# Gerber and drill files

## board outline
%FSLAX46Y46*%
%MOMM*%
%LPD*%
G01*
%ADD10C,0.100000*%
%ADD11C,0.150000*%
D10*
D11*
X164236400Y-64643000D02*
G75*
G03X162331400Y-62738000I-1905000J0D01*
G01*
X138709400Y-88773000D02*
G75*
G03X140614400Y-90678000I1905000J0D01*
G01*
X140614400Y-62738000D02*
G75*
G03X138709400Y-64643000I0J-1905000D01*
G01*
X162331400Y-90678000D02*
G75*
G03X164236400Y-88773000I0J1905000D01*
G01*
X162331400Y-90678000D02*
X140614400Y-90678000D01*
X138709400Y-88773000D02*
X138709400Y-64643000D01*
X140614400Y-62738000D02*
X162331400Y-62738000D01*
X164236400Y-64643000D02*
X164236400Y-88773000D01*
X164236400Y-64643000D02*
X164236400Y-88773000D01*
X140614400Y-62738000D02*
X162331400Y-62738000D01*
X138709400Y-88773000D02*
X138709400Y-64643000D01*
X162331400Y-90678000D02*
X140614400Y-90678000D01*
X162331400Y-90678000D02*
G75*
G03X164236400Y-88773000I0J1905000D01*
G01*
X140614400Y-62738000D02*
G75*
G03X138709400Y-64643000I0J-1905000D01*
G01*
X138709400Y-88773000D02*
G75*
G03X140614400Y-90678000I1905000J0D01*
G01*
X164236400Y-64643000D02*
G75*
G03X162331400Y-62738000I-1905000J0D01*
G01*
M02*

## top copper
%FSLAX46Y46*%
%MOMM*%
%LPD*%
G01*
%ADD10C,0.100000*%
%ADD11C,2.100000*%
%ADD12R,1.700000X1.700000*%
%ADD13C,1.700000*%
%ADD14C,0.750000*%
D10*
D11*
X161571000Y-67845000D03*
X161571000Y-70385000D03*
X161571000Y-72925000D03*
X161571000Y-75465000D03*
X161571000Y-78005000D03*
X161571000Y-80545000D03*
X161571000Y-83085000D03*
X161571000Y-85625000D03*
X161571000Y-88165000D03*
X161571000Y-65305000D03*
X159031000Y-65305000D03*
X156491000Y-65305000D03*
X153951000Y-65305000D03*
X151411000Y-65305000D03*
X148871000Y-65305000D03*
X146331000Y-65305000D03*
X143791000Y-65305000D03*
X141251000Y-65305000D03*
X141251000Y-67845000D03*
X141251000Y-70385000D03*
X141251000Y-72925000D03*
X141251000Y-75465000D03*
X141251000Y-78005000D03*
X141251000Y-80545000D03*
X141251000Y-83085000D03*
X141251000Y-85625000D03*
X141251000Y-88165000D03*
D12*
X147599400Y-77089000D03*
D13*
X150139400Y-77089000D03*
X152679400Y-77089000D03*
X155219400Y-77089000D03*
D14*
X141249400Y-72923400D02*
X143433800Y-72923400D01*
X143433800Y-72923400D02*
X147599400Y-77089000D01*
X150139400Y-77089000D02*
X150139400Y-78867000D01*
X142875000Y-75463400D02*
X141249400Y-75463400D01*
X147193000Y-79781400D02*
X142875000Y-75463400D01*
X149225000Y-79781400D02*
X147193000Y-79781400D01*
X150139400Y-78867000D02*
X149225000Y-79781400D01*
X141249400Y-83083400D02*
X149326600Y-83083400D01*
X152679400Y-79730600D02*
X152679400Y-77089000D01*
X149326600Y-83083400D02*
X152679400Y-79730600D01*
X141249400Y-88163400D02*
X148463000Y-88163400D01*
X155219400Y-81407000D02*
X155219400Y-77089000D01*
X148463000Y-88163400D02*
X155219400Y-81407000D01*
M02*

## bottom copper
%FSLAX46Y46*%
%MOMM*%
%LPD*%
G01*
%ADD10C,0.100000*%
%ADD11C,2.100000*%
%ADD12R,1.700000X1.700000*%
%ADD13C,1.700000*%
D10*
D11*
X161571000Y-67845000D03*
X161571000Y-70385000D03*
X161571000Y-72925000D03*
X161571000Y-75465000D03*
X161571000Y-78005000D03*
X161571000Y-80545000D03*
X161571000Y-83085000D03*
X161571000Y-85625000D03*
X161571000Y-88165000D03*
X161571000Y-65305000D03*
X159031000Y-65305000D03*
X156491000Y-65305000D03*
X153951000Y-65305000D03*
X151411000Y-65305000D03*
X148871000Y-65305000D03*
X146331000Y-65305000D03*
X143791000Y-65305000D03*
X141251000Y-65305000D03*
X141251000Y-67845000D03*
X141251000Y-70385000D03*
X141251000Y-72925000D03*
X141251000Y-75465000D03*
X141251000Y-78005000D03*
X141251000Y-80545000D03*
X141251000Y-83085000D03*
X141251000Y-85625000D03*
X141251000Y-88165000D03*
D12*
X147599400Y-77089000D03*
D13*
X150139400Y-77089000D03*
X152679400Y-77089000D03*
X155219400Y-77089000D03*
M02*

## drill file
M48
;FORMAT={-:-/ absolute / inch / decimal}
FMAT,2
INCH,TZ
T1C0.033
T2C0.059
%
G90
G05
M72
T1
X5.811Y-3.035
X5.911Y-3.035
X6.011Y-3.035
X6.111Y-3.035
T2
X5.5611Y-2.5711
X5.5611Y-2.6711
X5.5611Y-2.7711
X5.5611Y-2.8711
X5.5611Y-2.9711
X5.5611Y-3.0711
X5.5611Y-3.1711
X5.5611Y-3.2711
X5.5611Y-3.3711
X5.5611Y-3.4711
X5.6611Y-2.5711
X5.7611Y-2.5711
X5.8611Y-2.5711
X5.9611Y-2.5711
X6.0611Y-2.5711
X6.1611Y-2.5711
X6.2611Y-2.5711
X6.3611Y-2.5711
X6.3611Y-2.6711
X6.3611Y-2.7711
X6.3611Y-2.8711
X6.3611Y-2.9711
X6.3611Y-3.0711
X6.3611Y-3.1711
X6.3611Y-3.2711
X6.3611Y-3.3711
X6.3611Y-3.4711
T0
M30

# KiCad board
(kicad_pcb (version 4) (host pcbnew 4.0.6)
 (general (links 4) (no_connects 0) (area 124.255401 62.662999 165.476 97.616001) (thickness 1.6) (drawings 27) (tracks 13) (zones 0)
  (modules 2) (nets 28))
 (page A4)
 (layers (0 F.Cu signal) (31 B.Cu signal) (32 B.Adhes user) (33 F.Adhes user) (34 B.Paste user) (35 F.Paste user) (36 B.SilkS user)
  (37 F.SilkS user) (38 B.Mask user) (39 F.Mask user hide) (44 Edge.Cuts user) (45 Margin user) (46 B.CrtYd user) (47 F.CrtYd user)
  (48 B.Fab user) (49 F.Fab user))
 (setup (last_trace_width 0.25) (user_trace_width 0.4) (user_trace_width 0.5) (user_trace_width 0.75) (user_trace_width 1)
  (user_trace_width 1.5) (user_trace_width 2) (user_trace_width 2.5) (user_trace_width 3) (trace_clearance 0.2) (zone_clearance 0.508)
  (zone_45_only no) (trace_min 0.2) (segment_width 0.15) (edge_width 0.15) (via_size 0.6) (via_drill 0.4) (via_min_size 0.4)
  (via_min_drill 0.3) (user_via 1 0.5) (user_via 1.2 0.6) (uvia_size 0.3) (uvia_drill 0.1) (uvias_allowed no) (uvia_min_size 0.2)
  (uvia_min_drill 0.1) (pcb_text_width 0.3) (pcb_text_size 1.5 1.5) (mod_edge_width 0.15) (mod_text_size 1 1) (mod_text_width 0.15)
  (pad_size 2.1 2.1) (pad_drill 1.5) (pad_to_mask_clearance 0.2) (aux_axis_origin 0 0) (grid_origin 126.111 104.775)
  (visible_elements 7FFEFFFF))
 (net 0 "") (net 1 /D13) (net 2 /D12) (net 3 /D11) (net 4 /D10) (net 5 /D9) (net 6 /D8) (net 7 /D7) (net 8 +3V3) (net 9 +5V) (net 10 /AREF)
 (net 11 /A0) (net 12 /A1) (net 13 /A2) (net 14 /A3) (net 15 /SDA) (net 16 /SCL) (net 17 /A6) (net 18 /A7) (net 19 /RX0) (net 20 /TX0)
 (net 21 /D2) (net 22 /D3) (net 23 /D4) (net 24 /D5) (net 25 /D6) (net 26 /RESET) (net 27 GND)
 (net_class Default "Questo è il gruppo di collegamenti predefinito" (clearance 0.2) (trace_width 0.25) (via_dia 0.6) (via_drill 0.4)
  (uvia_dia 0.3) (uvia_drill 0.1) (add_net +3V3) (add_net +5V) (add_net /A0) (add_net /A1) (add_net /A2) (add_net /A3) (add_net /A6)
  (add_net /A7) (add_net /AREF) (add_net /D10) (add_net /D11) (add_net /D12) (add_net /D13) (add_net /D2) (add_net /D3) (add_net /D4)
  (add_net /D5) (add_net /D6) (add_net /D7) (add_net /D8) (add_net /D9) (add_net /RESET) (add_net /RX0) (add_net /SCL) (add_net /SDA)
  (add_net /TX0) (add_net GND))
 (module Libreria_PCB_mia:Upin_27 (layer B.Cu) (at 161.571 88.165 180)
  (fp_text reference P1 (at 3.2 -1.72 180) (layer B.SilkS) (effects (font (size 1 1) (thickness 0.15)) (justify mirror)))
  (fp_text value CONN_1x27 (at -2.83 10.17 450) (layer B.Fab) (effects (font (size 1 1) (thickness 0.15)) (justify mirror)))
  (pad 9 thru_hole circle (at 0 20.32 180) (size 2.1 2.1) (drill 1.5) (layers *.Cu *.Mask) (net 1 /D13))
  (pad 8 thru_hole circle (at 0 17.78 180) (size 2.1 2.1) (drill 1.5) (layers *.Cu *.Mask) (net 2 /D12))
  (pad 7 thru_hole circle (at 0 15.24 180) (size 2.1 2.1) (drill 1.5) (layers *.Cu *.Mask) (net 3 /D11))
  (pad 6 thru_hole circle (at 0 12.7 180) (size 2.1 2.1) (drill 1.5) (layers *.Cu *.Mask) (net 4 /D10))
  (pad 5 thru_hole circle (at 0 10.16 180) (size 2.1 2.1) (drill 1.5) (layers *.Cu *.Mask) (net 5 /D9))
  (pad 4 thru_hole circle (at 0 7.62 180) (size 2.1 2.1) (drill 1.5) (layers *.Cu *.Mask) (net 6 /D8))
  (pad 3 thru_hole circle (at 0 5.08 180) (size 2.1 2.1) (drill 1.5) (layers *.Cu *.Mask) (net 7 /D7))
  (pad 2 thru_hole circle (at 0 2.54 180) (size 2.1 2.1) (drill 1.5) (layers *.Cu *.Mask) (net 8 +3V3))
  (pad 1 thru_hole circle (at 0 0 180) (size 2.1 2.1) (drill 1.5) (layers *.Cu *.Mask) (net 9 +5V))
  (pad 10 thru_hole circle (at 0 22.86 180) (size 2.1 2.1) (drill 1.5) (layers *.Cu *.Mask) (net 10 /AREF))
  (pad 11 thru_hole circle (at 2.54 22.86 180) (size 2.1 2.1) (drill 1.5) (layers *.Cu *.Mask) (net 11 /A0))
  (pad 12 thru_hole circle (at 5.08 22.86 180) (size 2.1 2.1) (drill 1.5) (layers *.Cu *.Mask) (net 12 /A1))
  (pad 13 thru_hole circle (at 7.62 22.86 180) (size 2.1 2.1) (drill 1.5) (layers *.Cu *.Mask) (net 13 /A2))
  (pad 14 thru_hole circle (at 10.16 22.86 180) (size 2.1 2.1) (drill 1.5) (layers *.Cu *.Mask) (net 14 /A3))
  (pad 15 thru_hole circle (at 12.7 22.86 180) (size 2.1 2.1) (drill 1.5) (layers *.Cu *.Mask) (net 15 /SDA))
  (pad 16 thru_hole circle (at 15.24 22.86 180) (size 2.1 2.1) (drill 1.5) (layers *.Cu *.Mask) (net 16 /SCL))
  (pad 17 thru_hole circle (at 17.78 22.86 180) (size 2.1 2.1) (drill 1.5) (layers *.Cu *.Mask) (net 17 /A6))
  (pad 18 thru_hole circle (at 20.32 22.86 180) (size 2.1 2.1) (drill 1.5) (layers *.Cu *.Mask) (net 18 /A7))
  (pad 19 thru_hole circle (at 20.32 20.32 180) (size 2.1 2.1) (drill 1.5) (layers *.Cu *.Mask) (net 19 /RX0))
  (pad 20 thru_hole circle (at 20.32 17.78 180) (size 2.1 2.1) (drill 1.5) (layers *.Cu *.Mask) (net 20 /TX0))
  (pad 21 thru_hole circle (at 20.32 15.24 180) (size 2.1 2.1) (drill 1.5) (layers *.Cu *.Mask) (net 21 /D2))
  (pad 22 thru_hole circle (at 20.32 12.7 180) (size 2.1 2.1) (drill 1.5) (layers *.Cu *.Mask) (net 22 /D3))
  (pad 23 thru_hole circle (at 20.32 10.16 180) (size 2.1 2.1) (drill 1.5) (layers *.Cu *.Mask) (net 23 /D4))
  (pad 24 thru_hole circle (at 20.32 7.62 180) (size 2.1 2.1) (drill 1.5) (layers *.Cu *.Mask) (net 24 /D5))
  (pad 25 thru_hole circle (at 20.32 5.08 180) (size 2.1 2.1) (drill 1.5) (layers *.Cu *.Mask) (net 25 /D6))
  (pad 26 thru_hole circle (at 20.32 2.54 180) (size 2.1 2.1) (drill 1.5) (layers *.Cu *.Mask) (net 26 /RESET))
  (pad 27 thru_hole circle (at 20.32 0 180) (size 2.1 2.1) (drill 1.5) (layers *.Cu *.Mask) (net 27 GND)))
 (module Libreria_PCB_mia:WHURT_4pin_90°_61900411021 (layer F.Cu) (at 147.5994 77.089)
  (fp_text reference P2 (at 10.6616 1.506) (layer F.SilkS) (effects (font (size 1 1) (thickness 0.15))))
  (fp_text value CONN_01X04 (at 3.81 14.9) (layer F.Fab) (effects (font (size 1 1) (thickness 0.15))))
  (pad 1 thru_hole rect (at 0 0) (size 1.7 1.7) (drill 0.85) (layers *.Cu *.Mask) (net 21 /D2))
  (pad 2 thru_hole circle (at 2.54 0) (size 1.7 1.7) (drill 0.85) (layers *.Cu *.Mask) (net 22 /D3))
  (pad 3 thru_hole circle (at 5.08 0) (size 1.7 1.7) (drill 0.85) (layers *.Cu *.Mask) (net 25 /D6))
  (pad 4 thru_hole circle (at 7.62 0) (size 1.7 1.7) (drill 0.85) (layers *.Cu *.Mask) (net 27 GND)))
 (gr_arc (start 162.3314 64.643) (end 162.3314 62.738) (angle 90) (layer Edge.Cuts) (width 0.15))
 (gr_arc (start 140.6144 88.773) (end 140.6144 90.678) (angle 90) (layer Edge.Cuts) (width 0.15))
 (gr_arc (start 140.6144 64.643) (end 138.7094 64.643) (angle 90) (layer Edge.Cuts) (width 0.15))
 (gr_arc (start 162.3314 88.773) (end 164.2364 88.773) (angle 90) (layer Edge.Cuts) (width 0.15))
 (gr_line (start 162.3314 90.678) (end 140.6144 90.678) (angle 90) (layer Edge.Cuts) (width 0.15))
 (gr_line (start 138.7094 88.773) (end 138.7094 64.643) (angle 90) (layer Edge.Cuts) (width 0.15))
 (gr_line (start 140.6144 62.738) (end 162.3314 62.738) (angle 90) (layer Edge.Cuts) (width 0.15))
 (gr_line (start 164.2364 64.643) (end 164.2364 88.773) (angle 90) (layer Edge.Cuts) (width 0.15))
 (gr_line (start 164.2364 64.643) (end 164.2364 88.773) (angle 90) (layer Edge.Cuts) (width 0.15))
 (gr_line (start 140.6144 62.738) (end 162.3314 62.738) (angle 90) (layer Edge.Cuts) (width 0.15))
 (gr_line (start 138.7094 88.773) (end 138.7094 64.643) (angle 90) (layer Edge.Cuts) (width 0.15))
 (gr_line (start 162.3314 90.678) (end 140.6144 90.678) (angle 90) (layer Edge.Cuts) (width 0.15))
 (gr_arc (start 162.3314 88.773) (end 164.2364 88.773) (angle 90) (layer Edge.Cuts) (width 0.15))
 (gr_arc (start 140.6144 64.643) (end 138.7094 64.643) (angle 90) (layer Edge.Cuts) (width 0.15))
 (gr_arc (start 140.6144 88.773) (end 140.6144 90.678) (angle 90) (layer Edge.Cuts) (width 0.15))
 (gr_arc (start 162.3314 64.643) (end 162.3314 62.738) (angle 90) (layer Edge.Cuts) (width 0.15))
 (segment (start 141.2494 72.9234) (end 143.4338 72.9234) (width 0.75) (layer F.Cu) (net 21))
 (segment (start 143.4338 72.9234) (end 147.5994 77.089) (width 0.75) (layer F.Cu) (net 21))
 (segment (start 150.1394 77.089) (end 150.1394 78.867) (width 0.75) (layer F.Cu) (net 22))
 (segment (start 142.875 75.4634) (end 141.2494 75.4634) (width 0.75) (layer F.Cu) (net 22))
 (segment (start 147.193 79.7814) (end 142.875 75.4634) (width 0.75) (layer F.Cu) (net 22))
 (segment (start 149.225 79.7814) (end 147.193 79.7814) (width 0.75) (layer F.Cu) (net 22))
 (segment (start 150.1394 78.867) (end 149.225 79.7814) (width 0.75) (layer F.Cu) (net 22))
 (segment (start 141.2494 83.0834) (end 149.3266 83.0834) (width 0.75) (layer F.Cu) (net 25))
 (segment (start 152.6794 79.7306) (end 152.6794 77.089) (width 0.75) (layer F.Cu) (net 25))
 (segment (start 149.3266 83.0834) (end 152.6794 79.7306) (width 0.75) (layer F.Cu) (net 25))
 (segment (start 141.2494 88.1634) (end 148.463 88.1634) (width 0.75) (layer F.Cu) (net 27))
 (segment (start 155.2194 81.407) (end 155.2194 77.089) (width 0.75) (layer F.Cu) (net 27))
 (segment (start 148.463 88.1634) (end 155.2194 81.407) (width 0.75) (layer F.Cu) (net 27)))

